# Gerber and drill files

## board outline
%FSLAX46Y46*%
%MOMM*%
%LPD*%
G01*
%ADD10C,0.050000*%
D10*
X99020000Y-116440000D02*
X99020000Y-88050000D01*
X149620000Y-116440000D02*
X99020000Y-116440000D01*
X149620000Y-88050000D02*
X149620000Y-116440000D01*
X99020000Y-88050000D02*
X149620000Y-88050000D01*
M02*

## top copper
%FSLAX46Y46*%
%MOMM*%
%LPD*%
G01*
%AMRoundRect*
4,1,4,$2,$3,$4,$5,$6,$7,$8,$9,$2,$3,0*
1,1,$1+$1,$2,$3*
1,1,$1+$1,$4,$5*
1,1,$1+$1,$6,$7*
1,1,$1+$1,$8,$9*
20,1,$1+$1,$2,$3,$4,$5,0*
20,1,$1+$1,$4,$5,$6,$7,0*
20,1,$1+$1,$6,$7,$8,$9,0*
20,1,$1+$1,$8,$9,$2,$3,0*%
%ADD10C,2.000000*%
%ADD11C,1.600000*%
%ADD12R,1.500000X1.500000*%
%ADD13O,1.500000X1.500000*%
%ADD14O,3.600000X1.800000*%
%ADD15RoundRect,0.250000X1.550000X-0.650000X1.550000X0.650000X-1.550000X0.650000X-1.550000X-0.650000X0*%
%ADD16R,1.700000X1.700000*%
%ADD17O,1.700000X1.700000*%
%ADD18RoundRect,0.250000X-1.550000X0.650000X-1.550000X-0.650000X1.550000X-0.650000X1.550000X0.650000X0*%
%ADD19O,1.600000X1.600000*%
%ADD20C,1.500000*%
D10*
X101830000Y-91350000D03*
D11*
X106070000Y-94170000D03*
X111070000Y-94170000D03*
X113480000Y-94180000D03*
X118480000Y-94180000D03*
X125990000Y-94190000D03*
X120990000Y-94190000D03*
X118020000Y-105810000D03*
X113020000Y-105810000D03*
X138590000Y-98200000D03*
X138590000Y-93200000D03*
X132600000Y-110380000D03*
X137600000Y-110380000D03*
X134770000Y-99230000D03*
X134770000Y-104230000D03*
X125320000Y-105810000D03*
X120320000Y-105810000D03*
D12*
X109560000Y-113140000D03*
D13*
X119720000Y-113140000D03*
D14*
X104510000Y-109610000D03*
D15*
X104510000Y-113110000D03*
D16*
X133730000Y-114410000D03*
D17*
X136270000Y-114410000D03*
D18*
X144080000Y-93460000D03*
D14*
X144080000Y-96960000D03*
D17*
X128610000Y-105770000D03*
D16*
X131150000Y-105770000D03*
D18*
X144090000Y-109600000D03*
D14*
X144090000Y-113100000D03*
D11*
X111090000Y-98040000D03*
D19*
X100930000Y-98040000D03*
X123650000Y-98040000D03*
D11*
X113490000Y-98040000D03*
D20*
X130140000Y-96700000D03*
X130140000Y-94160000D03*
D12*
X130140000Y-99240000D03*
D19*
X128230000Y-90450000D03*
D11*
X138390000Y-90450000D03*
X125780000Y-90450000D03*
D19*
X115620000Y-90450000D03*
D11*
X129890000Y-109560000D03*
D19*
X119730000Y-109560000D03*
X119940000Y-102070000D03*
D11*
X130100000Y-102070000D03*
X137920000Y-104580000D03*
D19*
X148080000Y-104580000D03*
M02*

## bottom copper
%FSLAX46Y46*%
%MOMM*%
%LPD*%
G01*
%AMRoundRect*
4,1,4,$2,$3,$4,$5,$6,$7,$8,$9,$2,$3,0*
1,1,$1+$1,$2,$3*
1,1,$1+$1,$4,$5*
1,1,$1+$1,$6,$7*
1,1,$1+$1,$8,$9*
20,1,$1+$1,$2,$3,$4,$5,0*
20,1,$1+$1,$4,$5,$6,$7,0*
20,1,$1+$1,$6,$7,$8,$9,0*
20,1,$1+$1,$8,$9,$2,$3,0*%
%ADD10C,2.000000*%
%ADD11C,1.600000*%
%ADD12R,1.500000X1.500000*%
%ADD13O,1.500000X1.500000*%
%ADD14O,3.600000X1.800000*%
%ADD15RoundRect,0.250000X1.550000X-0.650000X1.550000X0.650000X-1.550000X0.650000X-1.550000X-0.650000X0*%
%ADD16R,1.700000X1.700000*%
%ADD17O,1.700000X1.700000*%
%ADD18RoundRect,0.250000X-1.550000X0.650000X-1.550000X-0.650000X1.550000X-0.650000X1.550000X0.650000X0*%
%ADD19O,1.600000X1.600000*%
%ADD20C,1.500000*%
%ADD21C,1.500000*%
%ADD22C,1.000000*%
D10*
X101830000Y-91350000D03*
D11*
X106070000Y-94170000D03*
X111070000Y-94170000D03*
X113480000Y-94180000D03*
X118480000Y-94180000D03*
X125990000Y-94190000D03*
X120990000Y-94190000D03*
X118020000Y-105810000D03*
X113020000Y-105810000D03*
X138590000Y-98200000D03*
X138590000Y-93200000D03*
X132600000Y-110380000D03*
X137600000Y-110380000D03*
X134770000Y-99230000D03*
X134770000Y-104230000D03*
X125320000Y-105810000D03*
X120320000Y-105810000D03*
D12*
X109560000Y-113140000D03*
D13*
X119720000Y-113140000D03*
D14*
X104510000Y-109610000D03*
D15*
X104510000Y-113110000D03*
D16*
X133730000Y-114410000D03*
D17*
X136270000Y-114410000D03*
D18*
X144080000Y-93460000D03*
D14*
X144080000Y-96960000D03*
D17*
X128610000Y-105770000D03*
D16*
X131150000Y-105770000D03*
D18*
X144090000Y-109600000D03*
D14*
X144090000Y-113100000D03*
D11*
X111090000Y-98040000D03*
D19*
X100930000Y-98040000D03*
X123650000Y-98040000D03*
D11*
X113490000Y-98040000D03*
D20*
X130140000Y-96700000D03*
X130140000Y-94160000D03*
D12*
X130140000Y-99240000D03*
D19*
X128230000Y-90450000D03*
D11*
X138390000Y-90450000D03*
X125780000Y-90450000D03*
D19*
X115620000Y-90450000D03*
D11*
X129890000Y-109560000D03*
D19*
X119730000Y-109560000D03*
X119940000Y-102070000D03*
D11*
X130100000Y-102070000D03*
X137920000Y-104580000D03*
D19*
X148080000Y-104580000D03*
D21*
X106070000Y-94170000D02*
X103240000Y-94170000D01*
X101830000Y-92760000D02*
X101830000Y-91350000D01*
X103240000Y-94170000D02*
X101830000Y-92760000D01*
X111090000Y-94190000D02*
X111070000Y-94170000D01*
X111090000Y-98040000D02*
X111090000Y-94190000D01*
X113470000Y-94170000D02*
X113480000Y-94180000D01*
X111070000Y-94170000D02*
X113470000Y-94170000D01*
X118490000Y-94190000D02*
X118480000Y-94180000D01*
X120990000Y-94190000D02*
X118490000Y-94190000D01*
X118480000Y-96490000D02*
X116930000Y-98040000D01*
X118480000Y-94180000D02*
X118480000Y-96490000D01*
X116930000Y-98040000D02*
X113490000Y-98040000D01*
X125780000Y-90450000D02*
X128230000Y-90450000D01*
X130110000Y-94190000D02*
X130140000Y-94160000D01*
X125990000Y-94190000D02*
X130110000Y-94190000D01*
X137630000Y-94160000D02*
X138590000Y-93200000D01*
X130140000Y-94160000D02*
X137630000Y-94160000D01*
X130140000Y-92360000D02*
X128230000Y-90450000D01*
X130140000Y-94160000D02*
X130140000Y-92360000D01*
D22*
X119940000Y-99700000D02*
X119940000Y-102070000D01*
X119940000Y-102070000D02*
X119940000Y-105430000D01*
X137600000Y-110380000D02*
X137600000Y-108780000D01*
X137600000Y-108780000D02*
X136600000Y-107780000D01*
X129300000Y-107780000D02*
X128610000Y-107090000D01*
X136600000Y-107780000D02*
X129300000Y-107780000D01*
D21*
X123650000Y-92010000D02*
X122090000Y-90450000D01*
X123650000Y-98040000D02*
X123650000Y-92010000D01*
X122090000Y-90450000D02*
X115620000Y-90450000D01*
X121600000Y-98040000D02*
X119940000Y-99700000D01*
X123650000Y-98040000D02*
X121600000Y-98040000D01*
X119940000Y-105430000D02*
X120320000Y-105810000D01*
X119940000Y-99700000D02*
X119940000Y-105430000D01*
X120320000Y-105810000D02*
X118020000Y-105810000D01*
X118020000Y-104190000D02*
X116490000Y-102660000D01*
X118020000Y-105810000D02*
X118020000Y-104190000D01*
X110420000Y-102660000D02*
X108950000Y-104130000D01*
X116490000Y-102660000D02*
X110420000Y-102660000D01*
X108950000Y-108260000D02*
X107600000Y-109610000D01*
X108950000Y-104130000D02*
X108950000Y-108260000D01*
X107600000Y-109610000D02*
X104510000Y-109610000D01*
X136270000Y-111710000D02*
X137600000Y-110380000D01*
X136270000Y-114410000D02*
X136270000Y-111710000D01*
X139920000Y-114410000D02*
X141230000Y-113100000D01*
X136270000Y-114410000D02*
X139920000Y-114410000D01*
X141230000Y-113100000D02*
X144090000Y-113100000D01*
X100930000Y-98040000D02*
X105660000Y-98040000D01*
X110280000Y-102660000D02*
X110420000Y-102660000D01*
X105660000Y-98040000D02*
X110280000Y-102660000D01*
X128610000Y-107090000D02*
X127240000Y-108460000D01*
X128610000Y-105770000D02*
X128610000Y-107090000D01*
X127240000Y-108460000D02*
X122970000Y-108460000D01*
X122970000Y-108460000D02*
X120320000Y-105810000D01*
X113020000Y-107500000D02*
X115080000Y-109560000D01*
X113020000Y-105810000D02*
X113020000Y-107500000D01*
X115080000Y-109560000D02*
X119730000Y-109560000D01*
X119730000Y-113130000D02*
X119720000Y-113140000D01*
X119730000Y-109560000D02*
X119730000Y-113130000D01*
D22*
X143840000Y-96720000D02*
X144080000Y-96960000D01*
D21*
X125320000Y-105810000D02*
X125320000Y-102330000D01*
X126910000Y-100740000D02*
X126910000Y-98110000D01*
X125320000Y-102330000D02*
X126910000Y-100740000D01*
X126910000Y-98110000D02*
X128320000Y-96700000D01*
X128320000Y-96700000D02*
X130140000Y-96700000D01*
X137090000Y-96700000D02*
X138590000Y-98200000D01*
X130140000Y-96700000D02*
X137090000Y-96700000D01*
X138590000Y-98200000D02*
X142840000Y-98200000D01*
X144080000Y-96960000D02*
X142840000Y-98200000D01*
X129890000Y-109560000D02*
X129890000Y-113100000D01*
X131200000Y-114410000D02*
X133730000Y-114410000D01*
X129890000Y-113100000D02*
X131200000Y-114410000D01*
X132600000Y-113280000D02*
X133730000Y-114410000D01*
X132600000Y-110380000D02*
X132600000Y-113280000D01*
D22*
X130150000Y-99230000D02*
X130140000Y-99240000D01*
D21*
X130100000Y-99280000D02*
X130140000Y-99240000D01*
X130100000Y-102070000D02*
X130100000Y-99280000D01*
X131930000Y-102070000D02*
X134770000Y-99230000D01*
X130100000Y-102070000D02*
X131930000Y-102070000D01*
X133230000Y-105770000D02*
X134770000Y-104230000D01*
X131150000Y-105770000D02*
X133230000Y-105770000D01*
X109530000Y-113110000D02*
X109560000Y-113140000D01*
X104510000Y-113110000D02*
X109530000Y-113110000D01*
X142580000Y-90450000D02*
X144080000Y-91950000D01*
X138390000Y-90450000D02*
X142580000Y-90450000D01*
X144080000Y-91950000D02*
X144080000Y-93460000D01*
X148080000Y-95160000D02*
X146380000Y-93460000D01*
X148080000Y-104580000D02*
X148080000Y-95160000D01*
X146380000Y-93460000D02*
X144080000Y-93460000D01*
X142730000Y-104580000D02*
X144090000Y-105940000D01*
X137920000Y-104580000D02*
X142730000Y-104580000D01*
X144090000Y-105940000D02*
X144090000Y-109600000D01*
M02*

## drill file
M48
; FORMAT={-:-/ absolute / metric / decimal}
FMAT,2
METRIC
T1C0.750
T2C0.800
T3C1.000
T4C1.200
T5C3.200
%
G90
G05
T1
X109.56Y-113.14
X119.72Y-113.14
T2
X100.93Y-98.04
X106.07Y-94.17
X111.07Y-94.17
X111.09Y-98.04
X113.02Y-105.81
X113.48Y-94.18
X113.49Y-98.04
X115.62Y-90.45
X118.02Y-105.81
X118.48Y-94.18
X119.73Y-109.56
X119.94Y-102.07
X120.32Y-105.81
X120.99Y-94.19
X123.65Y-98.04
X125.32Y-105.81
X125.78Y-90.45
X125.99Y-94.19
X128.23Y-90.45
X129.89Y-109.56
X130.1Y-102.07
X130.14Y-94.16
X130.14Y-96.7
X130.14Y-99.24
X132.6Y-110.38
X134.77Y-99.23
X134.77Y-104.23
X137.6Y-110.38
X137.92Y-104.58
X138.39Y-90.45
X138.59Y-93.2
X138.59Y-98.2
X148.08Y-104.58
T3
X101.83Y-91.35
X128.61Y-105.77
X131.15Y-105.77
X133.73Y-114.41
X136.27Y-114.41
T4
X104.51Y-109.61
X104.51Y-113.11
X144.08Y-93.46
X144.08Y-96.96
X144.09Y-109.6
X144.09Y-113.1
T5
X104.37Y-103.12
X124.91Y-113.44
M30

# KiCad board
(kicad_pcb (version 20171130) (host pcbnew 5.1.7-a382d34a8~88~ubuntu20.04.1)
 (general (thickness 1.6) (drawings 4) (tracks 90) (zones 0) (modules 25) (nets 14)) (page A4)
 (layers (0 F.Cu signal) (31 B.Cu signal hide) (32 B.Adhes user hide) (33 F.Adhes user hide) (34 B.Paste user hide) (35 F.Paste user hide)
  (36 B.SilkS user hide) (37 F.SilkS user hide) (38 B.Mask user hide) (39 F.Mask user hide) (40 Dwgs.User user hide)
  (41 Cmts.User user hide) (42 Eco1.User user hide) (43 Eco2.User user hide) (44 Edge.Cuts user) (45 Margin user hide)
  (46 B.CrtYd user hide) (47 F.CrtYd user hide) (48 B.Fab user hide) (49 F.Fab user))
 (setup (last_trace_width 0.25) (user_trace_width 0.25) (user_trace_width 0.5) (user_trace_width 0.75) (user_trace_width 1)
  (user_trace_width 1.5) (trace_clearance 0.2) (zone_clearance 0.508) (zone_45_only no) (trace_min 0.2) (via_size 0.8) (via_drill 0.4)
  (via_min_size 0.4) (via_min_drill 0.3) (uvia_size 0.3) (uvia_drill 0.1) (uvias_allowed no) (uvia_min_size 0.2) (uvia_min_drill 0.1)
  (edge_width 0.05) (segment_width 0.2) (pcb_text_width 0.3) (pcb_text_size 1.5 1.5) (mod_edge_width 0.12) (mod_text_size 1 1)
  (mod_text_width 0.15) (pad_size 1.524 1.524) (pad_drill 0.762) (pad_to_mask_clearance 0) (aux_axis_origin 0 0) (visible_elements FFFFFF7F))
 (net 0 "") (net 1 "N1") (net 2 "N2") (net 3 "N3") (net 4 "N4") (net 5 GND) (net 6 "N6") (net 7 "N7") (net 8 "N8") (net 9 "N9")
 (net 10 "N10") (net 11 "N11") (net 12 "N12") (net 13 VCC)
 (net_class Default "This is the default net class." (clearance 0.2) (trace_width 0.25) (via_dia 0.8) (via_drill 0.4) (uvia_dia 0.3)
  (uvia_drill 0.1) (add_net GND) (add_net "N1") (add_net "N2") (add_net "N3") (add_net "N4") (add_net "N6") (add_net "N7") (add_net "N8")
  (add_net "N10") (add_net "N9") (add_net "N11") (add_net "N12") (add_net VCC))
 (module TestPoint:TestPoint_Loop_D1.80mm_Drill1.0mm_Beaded (layer F.Cu) (at 101.83 91.35)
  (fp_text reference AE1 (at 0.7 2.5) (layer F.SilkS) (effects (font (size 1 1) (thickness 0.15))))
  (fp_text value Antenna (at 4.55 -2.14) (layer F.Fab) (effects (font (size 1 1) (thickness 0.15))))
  (pad 1 thru_hole circle (at 0 0) (size 2 2) (drill 1) (layers *.Cu *.Mask) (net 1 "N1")))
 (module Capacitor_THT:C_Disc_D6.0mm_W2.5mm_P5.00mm (layer F.Cu) (at 111.07 94.17 180)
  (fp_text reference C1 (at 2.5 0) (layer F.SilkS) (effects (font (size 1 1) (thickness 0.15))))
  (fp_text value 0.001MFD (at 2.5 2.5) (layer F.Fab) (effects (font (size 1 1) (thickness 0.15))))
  (pad 2 thru_hole circle (at 5 0 180) (size 1.6 1.6) (drill 0.8) (layers *.Cu *.Mask) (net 1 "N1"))
  (pad 1 thru_hole circle (at 0 0 180) (size 1.6 1.6) (drill 0.8) (layers *.Cu *.Mask) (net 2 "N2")))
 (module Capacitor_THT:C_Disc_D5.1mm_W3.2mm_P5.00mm (layer F.Cu) (at 118.48 94.18 180)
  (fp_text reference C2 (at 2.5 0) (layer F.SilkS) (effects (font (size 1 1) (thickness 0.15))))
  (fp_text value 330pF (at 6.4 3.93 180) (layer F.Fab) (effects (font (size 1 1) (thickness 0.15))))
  (pad 2 thru_hole circle (at 5 0 180) (size 1.6 1.6) (drill 0.8) (layers *.Cu *.Mask) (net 2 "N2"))
  (pad 1 thru_hole circle (at 0 0 180) (size 1.6 1.6) (drill 0.8) (layers *.Cu *.Mask) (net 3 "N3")))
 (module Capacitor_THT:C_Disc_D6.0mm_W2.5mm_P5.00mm (layer F.Cu) (at 125.99 94.19 180)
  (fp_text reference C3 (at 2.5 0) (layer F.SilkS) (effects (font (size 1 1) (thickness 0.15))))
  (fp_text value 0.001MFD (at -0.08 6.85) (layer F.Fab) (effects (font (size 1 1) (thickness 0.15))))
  (pad 1 thru_hole circle (at 0 0 180) (size 1.6 1.6) (drill 0.8) (layers *.Cu *.Mask) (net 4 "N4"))
  (pad 2 thru_hole circle (at 5 0 180) (size 1.6 1.6) (drill 0.8) (layers *.Cu *.Mask) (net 3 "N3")))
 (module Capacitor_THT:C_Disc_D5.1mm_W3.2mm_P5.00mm (layer F.Cu) (at 113.02 105.81)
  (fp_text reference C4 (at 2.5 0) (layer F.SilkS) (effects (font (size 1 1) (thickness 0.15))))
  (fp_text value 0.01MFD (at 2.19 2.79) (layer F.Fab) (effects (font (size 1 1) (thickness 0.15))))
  (pad 2 thru_hole circle (at 5 0) (size 1.6 1.6) (drill 0.8) (layers *.Cu *.Mask) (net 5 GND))
  (pad 1 thru_hole circle (at 0 0) (size 1.6 1.6) (drill 0.8) (layers *.Cu *.Mask) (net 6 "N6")))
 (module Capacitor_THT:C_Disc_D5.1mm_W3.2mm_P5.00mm (layer F.Cu) (at 138.59 98.2 90)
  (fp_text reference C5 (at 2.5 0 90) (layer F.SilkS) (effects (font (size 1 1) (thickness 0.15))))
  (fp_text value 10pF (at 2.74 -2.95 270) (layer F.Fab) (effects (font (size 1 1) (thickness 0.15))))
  (pad 1 thru_hole circle (at 0 0 90) (size 1.6 1.6) (drill 0.8) (layers *.Cu *.Mask) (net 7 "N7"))
  (pad 2 thru_hole circle (at 5 0 90) (size 1.6 1.6) (drill 0.8) (layers *.Cu *.Mask) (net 4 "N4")))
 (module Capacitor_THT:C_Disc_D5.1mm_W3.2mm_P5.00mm (layer F.Cu) (at 132.6 110.38)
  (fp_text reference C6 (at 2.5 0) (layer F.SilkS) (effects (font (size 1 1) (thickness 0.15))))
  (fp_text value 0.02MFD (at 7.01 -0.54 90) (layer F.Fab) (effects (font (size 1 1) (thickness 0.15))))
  (pad 1 thru_hole circle (at 0 0) (size 1.6 1.6) (drill 0.8) (layers *.Cu *.Mask) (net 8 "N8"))
  (pad 2 thru_hole circle (at 5 0) (size 1.6 1.6) (drill 0.8) (layers *.Cu *.Mask) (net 5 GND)))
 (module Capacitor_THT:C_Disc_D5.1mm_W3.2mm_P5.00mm (layer F.Cu) (at 134.77 104.23 90)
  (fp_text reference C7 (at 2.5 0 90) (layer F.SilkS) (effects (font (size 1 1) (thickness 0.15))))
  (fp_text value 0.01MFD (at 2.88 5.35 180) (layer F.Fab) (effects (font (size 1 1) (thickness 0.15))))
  (pad 2 thru_hole circle (at 5 0 90) (size 1.6 1.6) (drill 0.8) (layers *.Cu *.Mask) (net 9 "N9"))
  (pad 1 thru_hole circle (at 0 0 90) (size 1.6 1.6) (drill 0.8) (layers *.Cu *.Mask) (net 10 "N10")))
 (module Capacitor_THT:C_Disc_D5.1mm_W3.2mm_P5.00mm (layer F.Cu) (at 125.32 105.81 180)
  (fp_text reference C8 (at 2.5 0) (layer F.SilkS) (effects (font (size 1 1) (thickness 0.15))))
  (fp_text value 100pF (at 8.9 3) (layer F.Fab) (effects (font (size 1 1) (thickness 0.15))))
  (pad 1 thru_hole circle (at 0 0 180) (size 1.6 1.6) (drill 0.8) (layers *.Cu *.Mask) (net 7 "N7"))
  (pad 2 thru_hole circle (at 5 0 180) (size 1.6 1.6) (drill 0.8) (layers *.Cu *.Mask) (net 5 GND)))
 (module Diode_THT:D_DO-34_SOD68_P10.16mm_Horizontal (layer F.Cu) (at 109.56 113.14)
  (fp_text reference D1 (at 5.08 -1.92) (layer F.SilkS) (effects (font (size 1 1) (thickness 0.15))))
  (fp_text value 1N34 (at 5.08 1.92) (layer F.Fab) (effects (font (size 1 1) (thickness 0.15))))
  (pad 1 thru_hole rect (at 0 0) (size 1.5 1.5) (drill 0.75) (layers *.Cu *.Mask) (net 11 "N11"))
  (pad 2 thru_hole oval (at 10.16 0) (size 1.5 1.5) (drill 0.75) (layers *.Cu *.Mask) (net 6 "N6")))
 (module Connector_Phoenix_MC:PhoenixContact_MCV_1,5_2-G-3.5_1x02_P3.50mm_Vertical (layer F.Cu) (at 104.51 113.11 90)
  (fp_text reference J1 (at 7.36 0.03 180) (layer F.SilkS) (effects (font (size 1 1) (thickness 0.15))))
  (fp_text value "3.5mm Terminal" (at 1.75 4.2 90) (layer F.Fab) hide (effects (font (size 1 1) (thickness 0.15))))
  (pad 2 thru_hole oval (at 3.5 0 90) (size 1.8 3.6) (drill 1.2) (layers *.Cu *.Mask) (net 5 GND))
  (pad 1 thru_hole roundrect (at 0 0 90) (size 1.8 3.6) (drill 1.2) (layers *.Cu *.Mask) (roundrect_rratio 0.138889) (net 11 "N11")))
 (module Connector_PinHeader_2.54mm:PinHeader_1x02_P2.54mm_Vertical (layer F.Cu) (at 133.73 114.41 90)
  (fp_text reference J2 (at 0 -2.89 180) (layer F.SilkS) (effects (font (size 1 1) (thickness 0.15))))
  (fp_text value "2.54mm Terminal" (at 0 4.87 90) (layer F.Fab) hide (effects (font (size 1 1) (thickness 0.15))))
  (pad 1 thru_hole rect (at 0 0 90) (size 1.7 1.7) (drill 1) (layers *.Cu *.Mask) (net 8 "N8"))
  (pad 2 thru_hole oval (at 0 2.54 90) (size 1.7 1.7) (drill 1) (layers *.Cu *.Mask) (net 5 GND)))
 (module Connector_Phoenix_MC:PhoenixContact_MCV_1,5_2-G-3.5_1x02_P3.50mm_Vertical (layer F.Cu) (at 144.08 93.46 270)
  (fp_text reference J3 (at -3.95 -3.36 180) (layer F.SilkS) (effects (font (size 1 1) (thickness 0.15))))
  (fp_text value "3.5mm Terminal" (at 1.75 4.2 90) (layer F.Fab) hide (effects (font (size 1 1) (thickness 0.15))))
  (pad 1 thru_hole roundrect (at 0 0 270) (size 1.8 3.6) (drill 1.2) (layers *.Cu *.Mask) (roundrect_rratio 0.138889) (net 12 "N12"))
  (pad 2 thru_hole oval (at 3.5 0 270) (size 1.8 3.6) (drill 1.2) (layers *.Cu *.Mask) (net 7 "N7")))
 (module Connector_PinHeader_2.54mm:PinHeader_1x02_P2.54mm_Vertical (layer F.Cu) (at 131.15 105.77 270)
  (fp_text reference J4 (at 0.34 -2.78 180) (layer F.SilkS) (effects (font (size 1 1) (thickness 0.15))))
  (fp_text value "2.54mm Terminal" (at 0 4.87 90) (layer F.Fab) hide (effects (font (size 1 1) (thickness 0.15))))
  (pad 2 thru_hole oval (at 0 2.54 270) (size 1.7 1.7) (drill 1) (layers *.Cu *.Mask) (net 5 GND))
  (pad 1 thru_hole rect (at 0 0 270) (size 1.7 1.7) (drill 1) (layers *.Cu *.Mask) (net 10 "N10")))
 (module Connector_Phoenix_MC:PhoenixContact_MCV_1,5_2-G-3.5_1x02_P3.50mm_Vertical (layer F.Cu) (at 144.09 109.6 270)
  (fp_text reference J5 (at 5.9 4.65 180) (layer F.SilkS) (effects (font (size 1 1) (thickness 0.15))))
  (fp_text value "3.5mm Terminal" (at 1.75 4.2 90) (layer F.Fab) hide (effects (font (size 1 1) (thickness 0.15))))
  (pad 1 thru_hole roundrect (at 0 0 270) (size 1.8 3.6) (drill 1.2) (layers *.Cu *.Mask) (roundrect_rratio 0.138889) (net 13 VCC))
  (pad 2 thru_hole oval (at 3.5 0 270) (size 1.8 3.6) (drill 1.2) (layers *.Cu *.Mask) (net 5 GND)))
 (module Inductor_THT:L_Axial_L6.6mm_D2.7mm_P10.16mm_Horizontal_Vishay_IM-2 (layer F.Cu) (at 111.09 98.04 180)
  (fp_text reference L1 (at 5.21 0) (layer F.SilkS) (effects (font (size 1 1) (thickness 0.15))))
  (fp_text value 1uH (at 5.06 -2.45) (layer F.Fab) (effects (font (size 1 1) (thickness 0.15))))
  (pad 1 thru_hole circle (at 0 0 180) (size 1.6 1.6) (drill 0.8) (layers *.Cu *.Mask) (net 2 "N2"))
  (pad 2 thru_hole oval (at 10.16 0 180) (size 1.6 1.6) (drill 0.8) (layers *.Cu *.Mask) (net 5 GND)))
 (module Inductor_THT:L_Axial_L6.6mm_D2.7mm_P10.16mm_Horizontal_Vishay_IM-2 (layer F.Cu) (at 113.49 98.04)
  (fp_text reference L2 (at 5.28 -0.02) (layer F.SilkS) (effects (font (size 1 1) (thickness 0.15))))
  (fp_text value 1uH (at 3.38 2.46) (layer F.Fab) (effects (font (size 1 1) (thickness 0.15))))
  (pad 2 thru_hole oval (at 10.16 0) (size 1.6 1.6) (drill 0.8) (layers *.Cu *.Mask) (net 5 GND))
  (pad 1 thru_hole circle (at 0 0) (size 1.6 1.6) (drill 0.8) (layers *.Cu *.Mask) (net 3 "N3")))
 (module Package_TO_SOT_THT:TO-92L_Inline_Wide (layer F.Cu) (at 130.14 99.24 90)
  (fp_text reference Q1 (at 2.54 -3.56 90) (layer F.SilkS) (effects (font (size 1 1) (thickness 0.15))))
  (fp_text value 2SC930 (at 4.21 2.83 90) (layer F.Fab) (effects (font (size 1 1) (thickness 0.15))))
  (pad 2 thru_hole circle (at 2.54 0 90) (size 1.5 1.5) (drill 0.8) (layers *.Cu *.Mask) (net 7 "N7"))
  (pad 3 thru_hole circle (at 5.08 0 90) (size 1.5 1.5) (drill 0.8) (layers *.Cu *.Mask) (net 4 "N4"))
  (pad 1 thru_hole rect (at 0 0 90) (size 1.5 1.5) (drill 0.8) (layers *.Cu *.Mask) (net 9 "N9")))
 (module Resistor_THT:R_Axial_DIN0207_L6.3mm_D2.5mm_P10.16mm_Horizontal (layer F.Cu) (at 138.39 90.45 180)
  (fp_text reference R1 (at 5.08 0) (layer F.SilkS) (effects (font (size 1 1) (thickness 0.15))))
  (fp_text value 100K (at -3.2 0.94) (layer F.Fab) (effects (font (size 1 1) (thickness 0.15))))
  (pad 2 thru_hole oval (at 10.16 0 180) (size 1.6 1.6) (drill 0.8) (layers *.Cu *.Mask) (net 4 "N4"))
  (pad 1 thru_hole circle (at 0 0 180) (size 1.6 1.6) (drill 0.8) (layers *.Cu *.Mask) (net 12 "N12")))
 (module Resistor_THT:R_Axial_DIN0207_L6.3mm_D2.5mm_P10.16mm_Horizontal (layer F.Cu) (at 125.78 90.45 180)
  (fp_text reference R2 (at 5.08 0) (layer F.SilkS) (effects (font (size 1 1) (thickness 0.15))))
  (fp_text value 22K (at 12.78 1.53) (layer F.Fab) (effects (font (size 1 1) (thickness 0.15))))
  (pad 1 thru_hole circle (at 0 0 180) (size 1.6 1.6) (drill 0.8) (layers *.Cu *.Mask) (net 4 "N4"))
  (pad 2 thru_hole oval (at 10.16 0 180) (size 1.6 1.6) (drill 0.8) (layers *.Cu *.Mask) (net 5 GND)))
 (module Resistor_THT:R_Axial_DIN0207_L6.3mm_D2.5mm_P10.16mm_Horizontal (layer F.Cu) (at 129.89 109.56 180)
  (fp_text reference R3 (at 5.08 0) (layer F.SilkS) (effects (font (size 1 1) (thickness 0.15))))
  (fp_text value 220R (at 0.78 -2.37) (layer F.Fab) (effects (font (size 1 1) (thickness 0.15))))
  (pad 1 thru_hole circle (at 0 0 180) (size 1.6 1.6) (drill 0.8) (layers *.Cu *.Mask) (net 8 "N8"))
  (pad 2 thru_hole oval (at 10.16 0 180) (size 1.6 1.6) (drill 0.8) (layers *.Cu *.Mask) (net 6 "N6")))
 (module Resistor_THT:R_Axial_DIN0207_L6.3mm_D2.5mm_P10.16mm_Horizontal (layer F.Cu) (at 130.1 102.07 180)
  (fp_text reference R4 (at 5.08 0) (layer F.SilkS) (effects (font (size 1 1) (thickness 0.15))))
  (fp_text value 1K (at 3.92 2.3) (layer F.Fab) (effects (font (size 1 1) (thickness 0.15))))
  (pad 2 thru_hole oval (at 10.16 0 180) (size 1.6 1.6) (drill 0.8) (layers *.Cu *.Mask) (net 5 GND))
  (pad 1 thru_hole circle (at 0 0 180) (size 1.6 1.6) (drill 0.8) (layers *.Cu *.Mask) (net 9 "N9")))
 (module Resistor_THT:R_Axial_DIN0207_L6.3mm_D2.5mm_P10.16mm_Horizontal (layer F.Cu) (at 137.92 104.58)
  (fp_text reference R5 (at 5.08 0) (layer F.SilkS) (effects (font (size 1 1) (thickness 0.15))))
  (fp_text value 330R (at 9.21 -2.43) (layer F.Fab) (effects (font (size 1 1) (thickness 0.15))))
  (pad 1 thru_hole circle (at 0 0) (size 1.6 1.6) (drill 0.8) (layers *.Cu *.Mask) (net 13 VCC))
  (pad 2 thru_hole oval (at 10.16 0) (size 1.6 1.6) (drill 0.8) (layers *.Cu *.Mask) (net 12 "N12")))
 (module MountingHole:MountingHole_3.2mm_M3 (layer F.Cu) (at 124.91 113.44)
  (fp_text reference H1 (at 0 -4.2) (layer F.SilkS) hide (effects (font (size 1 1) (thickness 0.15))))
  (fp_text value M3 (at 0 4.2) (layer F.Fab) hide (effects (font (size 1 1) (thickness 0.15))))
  (pad 1 np_thru_hole circle (at 0 0) (size 3.2 3.2) (drill 3.2) (layers *.Cu *.Mask)))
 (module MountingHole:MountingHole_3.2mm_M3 (layer F.Cu) (at 104.37 103.12)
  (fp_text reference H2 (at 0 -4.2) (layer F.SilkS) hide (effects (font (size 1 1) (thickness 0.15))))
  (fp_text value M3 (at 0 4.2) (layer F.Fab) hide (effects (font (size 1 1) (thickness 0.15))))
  (pad 1 np_thru_hole circle (at 0 0) (size 3.2 3.2) (drill 3.2) (layers *.Cu *.Mask)))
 (gr_line (start 99.02 116.44) (end 99.02 88.05) (layer Edge.Cuts) (width 0.05))
 (gr_line (start 149.62 116.44) (end 99.02 116.44) (layer Edge.Cuts) (width 0.05))
 (gr_line (start 149.62 88.05) (end 149.62 116.44) (layer Edge.Cuts) (width 0.05))
 (gr_line (start 99.02 88.05) (end 149.62 88.05) (layer Edge.Cuts) (width 0.05))
 (segment (start 106.07 94.17) (end 103.24 94.17) (width 1.5) (layer B.Cu) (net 1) (status 10))
 (segment (start 101.83 92.76) (end 101.83 91.35) (width 1.5) (layer B.Cu) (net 1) (status 20))
 (segment (start 103.24 94.17) (end 101.83 92.76) (width 1.5) (layer B.Cu) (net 1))
 (segment (start 111.09 94.19) (end 111.07 94.17) (width 1.5) (layer B.Cu) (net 2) (status 30))
 (segment (start 111.09 98.04) (end 111.09 94.19) (width 1.5) (layer B.Cu) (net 2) (status 30))
 (segment (start 113.47 94.17) (end 113.48 94.18) (width 1.5) (layer B.Cu) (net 2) (status 30))
 (segment (start 111.07 94.17) (end 113.47 94.17) (width 1.5) (layer B.Cu) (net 2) (status 30))
 (segment (start 118.49 94.19) (end 118.48 94.18) (width 1.5) (layer B.Cu) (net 3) (status 30))
 (segment (start 120.99 94.19) (end 118.49 94.19) (width 1.5) (layer B.Cu) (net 3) (status 30))
 (segment (start 118.48 96.49) (end 116.93 98.04) (width 1.5) (layer B.Cu) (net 3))
 (segment (start 118.48 94.18) (end 118.48 96.49) (width 1.5) (layer B.Cu) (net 3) (status 10))
 (segment (start 116.93 98.04) (end 113.49 98.04) (width 1.5) (layer B.Cu) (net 3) (status 20))
 (segment (start 125.78 90.45) (end 128.23 90.45) (width 1.5) (layer B.Cu) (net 4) (status 30))
 (segment (start 130.11 94.19) (end 130.14 94.16) (width 1.5) (layer B.Cu) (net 4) (status 30))
 (segment (start 125.99 94.19) (end 130.11 94.19) (width 1.5) (layer B.Cu) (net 4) (status 30))
 (segment (start 137.63 94.16) (end 138.59 93.2) (width 1.5) (layer B.Cu) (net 4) (status 20))
 (segment (start 130.14 94.16) (end 137.63 94.16) (width 1.5) (layer B.Cu) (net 4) (status 10))
 (segment (start 130.14 92.36) (end 128.23 90.45) (width 1.5) (layer B.Cu) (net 4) (status 20))
 (segment (start 130.14 94.16) (end 130.14 92.36) (width 1.5) (layer B.Cu) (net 4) (status 10))
 (segment (start 119.94 99.7) (end 119.94 102.07) (width 1) (layer B.Cu) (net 5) (status 20))
 (segment (start 119.94 102.07) (end 119.94 105.43) (width 1) (layer B.Cu) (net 5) (status 30))
 (segment (start 137.6 110.38) (end 137.6 108.78) (width 1) (layer B.Cu) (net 5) (status 10))
 (segment (start 137.6 108.78) (end 136.6 107.78) (width 1) (layer B.Cu) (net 5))
 (segment (start 129.3 107.78) (end 128.61 107.09) (width 1) (layer B.Cu) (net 5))
 (segment (start 136.6 107.78) (end 129.3 107.78) (width 1) (layer B.Cu) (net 5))
 (segment (start 123.65 92.01) (end 122.09 90.45) (width 1.5) (layer B.Cu) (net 5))
 (segment (start 123.65 98.04) (end 123.65 92.01) (width 1.5) (layer B.Cu) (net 5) (status 10))
 (segment (start 122.09 90.45) (end 115.62 90.45) (width 1.5) (layer B.Cu) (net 5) (status 20))
 (segment (start 121.6 98.04) (end 119.94 99.7) (width 1.5) (layer B.Cu) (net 5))
 (segment (start 123.65 98.04) (end 121.6 98.04) (width 1.5) (layer B.Cu) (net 5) (status 10))
 (segment (start 119.94 105.43) (end 120.32 105.81) (width 1.5) (layer B.Cu) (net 5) (status 30))
 (segment (start 119.94 99.7) (end 119.94 105.43) (width 1.5) (layer B.Cu) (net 5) (status 20))
 (segment (start 120.32 105.81) (end 118.02 105.81) (width 1.5) (layer B.Cu) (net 5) (status 30))
 (segment (start 118.02 104.19) (end 116.49 102.66) (width 1.5) (layer B.Cu) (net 5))
 (segment (start 118.02 105.81) (end 118.02 104.19) (width 1.5) (layer B.Cu) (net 5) (status 10))
 (segment (start 110.42 102.66) (end 108.95 104.13) (width 1.5) (layer B.Cu) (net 5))
 (segment (start 116.49 102.66) (end 110.42 102.66) (width 1.5) (layer B.Cu) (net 5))
 (segment (start 108.95 108.26) (end 107.6 109.61) (width 1.5) (layer B.Cu) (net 5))
 (segment (start 108.95 104.13) (end 108.95 108.26) (width 1.5) (layer B.Cu) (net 5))
 (segment (start 107.6 109.61) (end 104.51 109.61) (width 1.5) (layer B.Cu) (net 5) (status 20))
 (segment (start 136.27 111.71) (end 137.6 110.38) (width 1.5) (layer B.Cu) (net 5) (status 20))
 (segment (start 136.27 114.41) (end 136.27 111.71) (width 1.5) (layer B.Cu) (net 5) (status 10))
 (segment (start 139.92 114.41) (end 141.23 113.1) (width 1.5) (layer B.Cu) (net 5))
 (segment (start 136.27 114.41) (end 139.92 114.41) (width 1.5) (layer B.Cu) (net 5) (status 10))
 (segment (start 141.23 113.1) (end 144.09 113.1) (width 1.5) (layer B.Cu) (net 5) (status 20))
 (segment (start 100.93 98.04) (end 105.66 98.04) (width 1.5) (layer B.Cu) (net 5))
 (segment (start 110.28 102.66) (end 110.42 102.66) (width 1.5) (layer B.Cu) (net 5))
 (segment (start 105.66 98.04) (end 110.28 102.66) (width 1.5) (layer B.Cu) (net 5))
 (segment (start 128.61 107.09) (end 127.24 108.46) (width 1.5) (layer B.Cu) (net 5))
 (segment (start 128.61 105.77) (end 128.61 107.09) (width 1.5) (layer B.Cu) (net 5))
 (segment (start 127.24 108.46) (end 122.97 108.46) (width 1.5) (layer B.Cu) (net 5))
 (segment (start 122.97 108.46) (end 120.32 105.81) (width 1.5) (layer B.Cu) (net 5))
 (segment (start 113.02 107.5) (end 115.08 109.56) (width 1.5) (layer B.Cu) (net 6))
 (segment (start 113.02 105.81) (end 113.02 107.5) (width 1.5) (layer B.Cu) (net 6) (status 10))
 (segment (start 115.08 109.56) (end 119.73 109.56) (width 1.5) (layer B.Cu) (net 6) (status 20))
 (segment (start 119.73 113.13) (end 119.72 113.14) (width 1.5) (layer B.Cu) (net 6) (status 30))
 (segment (start 119.73 109.56) (end 119.73 113.13) (width 1.5) (layer B.Cu) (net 6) (status 30))
 (segment (start 143.84 96.72) (end 144.08 96.96) (width 1) (layer B.Cu) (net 7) (status 30))
 (segment (start 125.32 105.81) (end 125.32 102.33) (width 1.5) (layer B.Cu) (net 7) (status 10))
 (segment (start 126.91 100.74) (end 126.91 98.11) (width 1.5) (layer B.Cu) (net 7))
 (segment (start 125.32 102.33) (end 126.91 100.74) (width 1.5) (layer B.Cu) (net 7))
 (segment (start 126.91 98.11) (end 128.32 96.7) (width 1.5) (layer B.Cu) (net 7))
 (segment (start 128.32 96.7) (end 130.14 96.7) (width 1.5) (layer B.Cu) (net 7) (status 20))
 (segment (start 137.09 96.7) (end 138.59 98.2) (width 1.5) (layer B.Cu) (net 7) (status 20))
 (segment (start 130.14 96.7) (end 137.09 96.7) (width 1.5) (layer B.Cu) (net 7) (status 10))
 (segment (start 138.59 98.2) (end 142.84 98.2) (width 1.5) (layer B.Cu) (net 7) (status 10))
 (segment (start 144.08 96.96) (end 142.84 98.2) (width 1.5) (layer B.Cu) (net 7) (status 10))
 (segment (start 129.89 109.56) (end 129.89 113.1) (width 1.5) (layer B.Cu) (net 8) (status 10))
 (segment (start 131.2 114.41) (end 133.73 114.41) (width 1.5) (layer B.Cu) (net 8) (status 20))
 (segment (start 129.89 113.1) (end 131.2 114.41) (width 1.5) (layer B.Cu) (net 8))
 (segment (start 132.6 113.28) (end 133.73 114.41) (width 1.5) (layer B.Cu) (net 8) (status 20))
 (segment (start 132.6 110.38) (end 132.6 113.28) (width 1.5) (layer B.Cu) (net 8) (status 10))
 (segment (start 130.15 99.23) (end 130.14 99.24) (width 1) (layer B.Cu) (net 9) (status 30))
 (segment (start 130.1 99.28) (end 130.14 99.24) (width 1.5) (layer B.Cu) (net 9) (status 30))
 (segment (start 130.1 102.07) (end 130.1 99.28) (width 1.5) (layer B.Cu) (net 9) (status 30))
 (segment (start 131.93 102.07) (end 134.77 99.23) (width 1.5) (layer B.Cu) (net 9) (status 20))
 (segment (start 130.1 102.07) (end 131.93 102.07) (width 1.5) (layer B.Cu) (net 9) (status 10))
 (segment (start 133.23 105.77) (end 134.77 104.23) (width 1.5) (layer B.Cu) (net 10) (status 20))
 (segment (start 131.15 105.77) (end 133.23 105.77) (width 1.5) (layer B.Cu) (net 10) (status 10))
 (segment (start 109.53 113.11) (end 109.56 113.14) (width 1.5) (layer B.Cu) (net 11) (status 30))
 (segment (start 104.51 113.11) (end 109.53 113.11) (width 1.5) (layer B.Cu) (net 11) (status 30))
 (segment (start 142.58 90.45) (end 144.08 91.95) (width 1.5) (layer B.Cu) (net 12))
 (segment (start 138.39 90.45) (end 142.58 90.45) (width 1.5) (layer B.Cu) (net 12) (status 10))
 (segment (start 144.08 91.95) (end 144.08 93.46) (width 1.5) (layer B.Cu) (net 12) (status 20))
 (segment (start 148.08 95.16) (end 146.38 93.46) (width 1.5) (layer B.Cu) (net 12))
 (segment (start 148.08 104.58) (end 148.08 95.16) (width 1.5) (layer B.Cu) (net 12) (status 10))
 (segment (start 146.38 93.46) (end 144.08 93.46) (width 1.5) (layer B.Cu) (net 12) (status 20))
 (segment (start 142.73 104.58) (end 144.09 105.94) (width 1.5) (layer B.Cu) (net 13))
 (segment (start 137.92 104.58) (end 142.73 104.58) (width 1.5) (layer B.Cu) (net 13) (status 10))
 (segment (start 144.09 105.94) (end 144.09 109.6) (width 1.5) (layer B.Cu) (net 13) (status 20)))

